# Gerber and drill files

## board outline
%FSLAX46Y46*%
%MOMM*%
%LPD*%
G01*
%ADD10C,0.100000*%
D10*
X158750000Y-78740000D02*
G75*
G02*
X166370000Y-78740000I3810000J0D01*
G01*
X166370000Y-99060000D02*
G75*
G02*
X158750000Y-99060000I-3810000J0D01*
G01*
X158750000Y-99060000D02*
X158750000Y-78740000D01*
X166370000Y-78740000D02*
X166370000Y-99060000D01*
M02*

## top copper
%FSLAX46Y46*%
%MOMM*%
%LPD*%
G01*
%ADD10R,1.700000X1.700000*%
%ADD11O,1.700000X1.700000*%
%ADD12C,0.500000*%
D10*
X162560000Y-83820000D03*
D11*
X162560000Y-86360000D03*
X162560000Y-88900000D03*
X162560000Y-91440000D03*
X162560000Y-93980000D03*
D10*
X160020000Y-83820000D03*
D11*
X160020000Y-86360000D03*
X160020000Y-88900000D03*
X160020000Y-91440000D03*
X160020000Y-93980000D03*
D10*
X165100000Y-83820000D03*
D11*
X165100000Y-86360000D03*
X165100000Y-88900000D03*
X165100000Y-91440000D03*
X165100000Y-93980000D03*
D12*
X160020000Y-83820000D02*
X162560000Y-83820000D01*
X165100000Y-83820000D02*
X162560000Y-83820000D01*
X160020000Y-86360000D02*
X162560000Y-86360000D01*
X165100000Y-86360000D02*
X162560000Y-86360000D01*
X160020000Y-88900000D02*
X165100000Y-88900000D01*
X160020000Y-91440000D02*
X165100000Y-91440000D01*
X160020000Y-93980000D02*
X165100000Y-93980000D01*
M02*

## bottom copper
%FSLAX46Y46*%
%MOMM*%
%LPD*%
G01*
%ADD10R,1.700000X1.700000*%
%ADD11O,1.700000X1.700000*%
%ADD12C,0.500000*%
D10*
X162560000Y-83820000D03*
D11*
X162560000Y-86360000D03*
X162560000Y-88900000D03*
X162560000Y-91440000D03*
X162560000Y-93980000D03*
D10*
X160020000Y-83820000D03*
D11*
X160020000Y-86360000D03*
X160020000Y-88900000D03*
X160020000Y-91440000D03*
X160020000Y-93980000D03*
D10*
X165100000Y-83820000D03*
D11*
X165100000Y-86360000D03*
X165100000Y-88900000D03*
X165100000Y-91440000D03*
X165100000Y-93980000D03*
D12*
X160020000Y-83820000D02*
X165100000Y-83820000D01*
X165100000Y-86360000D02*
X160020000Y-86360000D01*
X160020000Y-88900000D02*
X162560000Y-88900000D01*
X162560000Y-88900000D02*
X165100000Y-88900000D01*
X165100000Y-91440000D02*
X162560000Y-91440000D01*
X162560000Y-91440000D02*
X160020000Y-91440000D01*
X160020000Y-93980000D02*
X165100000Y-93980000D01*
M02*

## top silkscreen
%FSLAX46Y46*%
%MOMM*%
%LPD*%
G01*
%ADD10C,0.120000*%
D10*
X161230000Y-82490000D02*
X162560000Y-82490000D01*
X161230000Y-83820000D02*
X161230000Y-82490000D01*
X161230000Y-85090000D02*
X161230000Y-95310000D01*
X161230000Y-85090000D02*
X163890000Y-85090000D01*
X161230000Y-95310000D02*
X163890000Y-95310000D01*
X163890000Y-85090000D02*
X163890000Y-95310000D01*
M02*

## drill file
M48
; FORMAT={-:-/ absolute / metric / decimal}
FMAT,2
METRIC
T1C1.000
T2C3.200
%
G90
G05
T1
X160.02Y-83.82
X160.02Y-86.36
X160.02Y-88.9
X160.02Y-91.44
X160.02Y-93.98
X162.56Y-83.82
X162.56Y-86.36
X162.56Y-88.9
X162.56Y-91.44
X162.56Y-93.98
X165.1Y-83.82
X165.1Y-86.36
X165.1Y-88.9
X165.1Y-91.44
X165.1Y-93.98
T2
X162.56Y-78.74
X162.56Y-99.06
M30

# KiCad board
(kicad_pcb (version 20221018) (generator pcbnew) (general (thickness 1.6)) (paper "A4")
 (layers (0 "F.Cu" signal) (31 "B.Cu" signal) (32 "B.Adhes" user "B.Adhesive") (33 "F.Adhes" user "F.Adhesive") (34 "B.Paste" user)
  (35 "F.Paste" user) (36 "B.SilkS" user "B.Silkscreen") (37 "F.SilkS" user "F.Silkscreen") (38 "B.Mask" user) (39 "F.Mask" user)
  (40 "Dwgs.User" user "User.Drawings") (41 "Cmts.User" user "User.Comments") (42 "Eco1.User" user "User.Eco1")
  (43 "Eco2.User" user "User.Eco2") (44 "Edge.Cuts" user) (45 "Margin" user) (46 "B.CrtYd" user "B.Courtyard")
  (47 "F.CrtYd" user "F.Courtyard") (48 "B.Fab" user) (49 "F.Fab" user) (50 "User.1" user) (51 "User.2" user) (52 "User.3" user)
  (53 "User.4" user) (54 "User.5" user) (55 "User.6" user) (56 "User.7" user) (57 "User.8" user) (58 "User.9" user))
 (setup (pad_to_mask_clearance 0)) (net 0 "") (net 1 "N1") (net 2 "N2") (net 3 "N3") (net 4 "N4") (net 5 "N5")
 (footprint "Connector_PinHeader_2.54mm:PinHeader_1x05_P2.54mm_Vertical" (layer "F.Cu") (at 162.56 83.82)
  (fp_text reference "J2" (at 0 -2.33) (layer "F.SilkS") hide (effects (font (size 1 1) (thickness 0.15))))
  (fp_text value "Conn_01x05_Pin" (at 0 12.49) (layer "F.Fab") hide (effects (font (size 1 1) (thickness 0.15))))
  (fp_line (start -1.33 -1.33) (end 0 -1.33) (stroke (width 0.12) (type solid)) (layer "F.SilkS"))
  (fp_line (start -1.33 0) (end -1.33 -1.33) (stroke (width 0.12) (type solid)) (layer "F.SilkS"))
  (fp_line (start -1.33 1.27) (end -1.33 11.49) (stroke (width 0.12) (type solid)) (layer "F.SilkS"))
  (fp_line (start -1.33 1.27) (end 1.33 1.27) (stroke (width 0.12) (type solid)) (layer "F.SilkS"))
  (fp_line (start -1.33 11.49) (end 1.33 11.49) (stroke (width 0.12) (type solid)) (layer "F.SilkS"))
  (fp_line (start 1.33 1.27) (end 1.33 11.49) (stroke (width 0.12) (type solid)) (layer "F.SilkS"))
  (pad "1" thru_hole rect (at 0 0) (size 1.7 1.7) (drill 1) (layers "*.Cu" "*.Mask") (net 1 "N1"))
  (pad "2" thru_hole oval (at 0 2.54) (size 1.7 1.7) (drill 1) (layers "*.Cu" "*.Mask") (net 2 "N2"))
  (pad "3" thru_hole oval (at 0 5.08) (size 1.7 1.7) (drill 1) (layers "*.Cu" "*.Mask") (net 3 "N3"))
  (pad "4" thru_hole oval (at 0 7.62) (size 1.7 1.7) (drill 1) (layers "*.Cu" "*.Mask") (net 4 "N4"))
  (pad "5" thru_hole oval (at 0 10.16) (size 1.7 1.7) (drill 1) (layers "*.Cu" "*.Mask") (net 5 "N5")))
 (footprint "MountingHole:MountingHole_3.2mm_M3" (layer "F.Cu") (at 162.56 78.74)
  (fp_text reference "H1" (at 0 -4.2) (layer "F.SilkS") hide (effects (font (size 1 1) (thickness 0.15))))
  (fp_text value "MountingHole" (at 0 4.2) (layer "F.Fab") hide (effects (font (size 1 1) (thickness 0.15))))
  (pad "" np_thru_hole circle (at 0 0) (size 3.2 3.2) (drill 3.2) (layers "*.Cu" "*.Mask")))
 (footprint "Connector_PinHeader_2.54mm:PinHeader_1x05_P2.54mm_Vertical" (layer "F.Cu") (at 160.02 83.82)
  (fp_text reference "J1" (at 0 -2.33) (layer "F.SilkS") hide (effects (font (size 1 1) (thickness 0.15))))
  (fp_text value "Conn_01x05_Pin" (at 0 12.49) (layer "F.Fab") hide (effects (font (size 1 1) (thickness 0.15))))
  (pad "1" thru_hole rect (at 0 0) (size 1.7 1.7) (drill 1) (layers "*.Cu" "*.Mask") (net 1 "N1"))
  (pad "2" thru_hole oval (at 0 2.54) (size 1.7 1.7) (drill 1) (layers "*.Cu" "*.Mask") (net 2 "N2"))
  (pad "3" thru_hole oval (at 0 5.08) (size 1.7 1.7) (drill 1) (layers "*.Cu" "*.Mask") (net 3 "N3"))
  (pad "4" thru_hole oval (at 0 7.62) (size 1.7 1.7) (drill 1) (layers "*.Cu" "*.Mask") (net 4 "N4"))
  (pad "5" thru_hole oval (at 0 10.16) (size 1.7 1.7) (drill 1) (layers "*.Cu" "*.Mask") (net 5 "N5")))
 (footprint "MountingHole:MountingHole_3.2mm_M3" (layer "F.Cu") (at 162.56 99.06)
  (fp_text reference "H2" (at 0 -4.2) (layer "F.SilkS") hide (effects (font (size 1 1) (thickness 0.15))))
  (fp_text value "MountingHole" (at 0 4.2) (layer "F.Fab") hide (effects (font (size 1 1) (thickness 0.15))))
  (pad "" np_thru_hole circle (at 0 0) (size 3.2 3.2) (drill 3.2) (layers "*.Cu" "*.Mask")))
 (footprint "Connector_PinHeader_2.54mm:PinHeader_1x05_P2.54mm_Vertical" (layer "F.Cu") (at 165.1 83.82)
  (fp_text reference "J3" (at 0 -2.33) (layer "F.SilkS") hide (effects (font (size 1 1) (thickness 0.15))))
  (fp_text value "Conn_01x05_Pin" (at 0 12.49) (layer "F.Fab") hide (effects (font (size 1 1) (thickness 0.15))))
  (pad "1" thru_hole rect (at 0 0) (size 1.7 1.7) (drill 1) (layers "*.Cu" "*.Mask") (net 1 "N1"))
  (pad "2" thru_hole oval (at 0 2.54) (size 1.7 1.7) (drill 1) (layers "*.Cu" "*.Mask") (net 2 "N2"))
  (pad "3" thru_hole oval (at 0 5.08) (size 1.7 1.7) (drill 1) (layers "*.Cu" "*.Mask") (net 3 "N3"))
  (pad "4" thru_hole oval (at 0 7.62) (size 1.7 1.7) (drill 1) (layers "*.Cu" "*.Mask") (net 4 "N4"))
  (pad "5" thru_hole oval (at 0 10.16) (size 1.7 1.7) (drill 1) (layers "*.Cu" "*.Mask") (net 5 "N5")))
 (gr_arc (start 158.75 78.74) (mid 162.56 74.93) (end 166.37 78.74) (stroke (width 0.1) (type default)) (layer "Edge.Cuts"))
 (gr_arc (start 166.37 99.06) (mid 162.56 102.87) (end 158.75 99.06) (stroke (width 0.1) (type default)) (layer "Edge.Cuts"))
 (gr_line (start 158.75 99.06) (end 158.75 78.74) (stroke (width 0.1) (type default)) (layer "Edge.Cuts"))
 (gr_line (start 166.37 78.74) (end 166.37 99.06) (stroke (width 0.1) (type default)) (layer "Edge.Cuts"))
 (segment (start 160.02 83.82) (end 162.56 83.82) (width 0.5) (layer "F.Cu") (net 1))
 (segment (start 165.1 83.82) (end 162.56 83.82) (width 0.5) (layer "F.Cu") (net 1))
 (segment (start 160.02 83.82) (end 165.1 83.82) (width 0.5) (layer "B.Cu") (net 1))
 (segment (start 160.02 86.36) (end 162.56 86.36) (width 0.5) (layer "F.Cu") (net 2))
 (segment (start 165.1 86.36) (end 162.56 86.36) (width 0.5) (layer "F.Cu") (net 2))
 (segment (start 165.1 86.36) (end 160.02 86.36) (width 0.5) (layer "B.Cu") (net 2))
 (segment (start 160.02 88.9) (end 165.1 88.9) (width 0.5) (layer "F.Cu") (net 3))
 (segment (start 160.02 88.9) (end 162.56 88.9) (width 0.5) (layer "B.Cu") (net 3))
 (segment (start 162.56 88.9) (end 165.1 88.9) (width 0.5) (layer "B.Cu") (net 3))
 (segment (start 160.02 91.44) (end 165.1 91.44) (width 0.5) (layer "F.Cu") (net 4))
 (segment (start 165.1 91.44) (end 162.56 91.44) (width 0.5) (layer "B.Cu") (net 4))
 (segment (start 162.56 91.44) (end 160.02 91.44) (width 0.5) (layer "B.Cu") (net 4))
 (segment (start 160.02 93.98) (end 165.1 93.98) (width 0.5) (layer "F.Cu") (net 5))
 (segment (start 160.02 93.98) (end 165.1 93.98) (width 0.5) (layer "B.Cu") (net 5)))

